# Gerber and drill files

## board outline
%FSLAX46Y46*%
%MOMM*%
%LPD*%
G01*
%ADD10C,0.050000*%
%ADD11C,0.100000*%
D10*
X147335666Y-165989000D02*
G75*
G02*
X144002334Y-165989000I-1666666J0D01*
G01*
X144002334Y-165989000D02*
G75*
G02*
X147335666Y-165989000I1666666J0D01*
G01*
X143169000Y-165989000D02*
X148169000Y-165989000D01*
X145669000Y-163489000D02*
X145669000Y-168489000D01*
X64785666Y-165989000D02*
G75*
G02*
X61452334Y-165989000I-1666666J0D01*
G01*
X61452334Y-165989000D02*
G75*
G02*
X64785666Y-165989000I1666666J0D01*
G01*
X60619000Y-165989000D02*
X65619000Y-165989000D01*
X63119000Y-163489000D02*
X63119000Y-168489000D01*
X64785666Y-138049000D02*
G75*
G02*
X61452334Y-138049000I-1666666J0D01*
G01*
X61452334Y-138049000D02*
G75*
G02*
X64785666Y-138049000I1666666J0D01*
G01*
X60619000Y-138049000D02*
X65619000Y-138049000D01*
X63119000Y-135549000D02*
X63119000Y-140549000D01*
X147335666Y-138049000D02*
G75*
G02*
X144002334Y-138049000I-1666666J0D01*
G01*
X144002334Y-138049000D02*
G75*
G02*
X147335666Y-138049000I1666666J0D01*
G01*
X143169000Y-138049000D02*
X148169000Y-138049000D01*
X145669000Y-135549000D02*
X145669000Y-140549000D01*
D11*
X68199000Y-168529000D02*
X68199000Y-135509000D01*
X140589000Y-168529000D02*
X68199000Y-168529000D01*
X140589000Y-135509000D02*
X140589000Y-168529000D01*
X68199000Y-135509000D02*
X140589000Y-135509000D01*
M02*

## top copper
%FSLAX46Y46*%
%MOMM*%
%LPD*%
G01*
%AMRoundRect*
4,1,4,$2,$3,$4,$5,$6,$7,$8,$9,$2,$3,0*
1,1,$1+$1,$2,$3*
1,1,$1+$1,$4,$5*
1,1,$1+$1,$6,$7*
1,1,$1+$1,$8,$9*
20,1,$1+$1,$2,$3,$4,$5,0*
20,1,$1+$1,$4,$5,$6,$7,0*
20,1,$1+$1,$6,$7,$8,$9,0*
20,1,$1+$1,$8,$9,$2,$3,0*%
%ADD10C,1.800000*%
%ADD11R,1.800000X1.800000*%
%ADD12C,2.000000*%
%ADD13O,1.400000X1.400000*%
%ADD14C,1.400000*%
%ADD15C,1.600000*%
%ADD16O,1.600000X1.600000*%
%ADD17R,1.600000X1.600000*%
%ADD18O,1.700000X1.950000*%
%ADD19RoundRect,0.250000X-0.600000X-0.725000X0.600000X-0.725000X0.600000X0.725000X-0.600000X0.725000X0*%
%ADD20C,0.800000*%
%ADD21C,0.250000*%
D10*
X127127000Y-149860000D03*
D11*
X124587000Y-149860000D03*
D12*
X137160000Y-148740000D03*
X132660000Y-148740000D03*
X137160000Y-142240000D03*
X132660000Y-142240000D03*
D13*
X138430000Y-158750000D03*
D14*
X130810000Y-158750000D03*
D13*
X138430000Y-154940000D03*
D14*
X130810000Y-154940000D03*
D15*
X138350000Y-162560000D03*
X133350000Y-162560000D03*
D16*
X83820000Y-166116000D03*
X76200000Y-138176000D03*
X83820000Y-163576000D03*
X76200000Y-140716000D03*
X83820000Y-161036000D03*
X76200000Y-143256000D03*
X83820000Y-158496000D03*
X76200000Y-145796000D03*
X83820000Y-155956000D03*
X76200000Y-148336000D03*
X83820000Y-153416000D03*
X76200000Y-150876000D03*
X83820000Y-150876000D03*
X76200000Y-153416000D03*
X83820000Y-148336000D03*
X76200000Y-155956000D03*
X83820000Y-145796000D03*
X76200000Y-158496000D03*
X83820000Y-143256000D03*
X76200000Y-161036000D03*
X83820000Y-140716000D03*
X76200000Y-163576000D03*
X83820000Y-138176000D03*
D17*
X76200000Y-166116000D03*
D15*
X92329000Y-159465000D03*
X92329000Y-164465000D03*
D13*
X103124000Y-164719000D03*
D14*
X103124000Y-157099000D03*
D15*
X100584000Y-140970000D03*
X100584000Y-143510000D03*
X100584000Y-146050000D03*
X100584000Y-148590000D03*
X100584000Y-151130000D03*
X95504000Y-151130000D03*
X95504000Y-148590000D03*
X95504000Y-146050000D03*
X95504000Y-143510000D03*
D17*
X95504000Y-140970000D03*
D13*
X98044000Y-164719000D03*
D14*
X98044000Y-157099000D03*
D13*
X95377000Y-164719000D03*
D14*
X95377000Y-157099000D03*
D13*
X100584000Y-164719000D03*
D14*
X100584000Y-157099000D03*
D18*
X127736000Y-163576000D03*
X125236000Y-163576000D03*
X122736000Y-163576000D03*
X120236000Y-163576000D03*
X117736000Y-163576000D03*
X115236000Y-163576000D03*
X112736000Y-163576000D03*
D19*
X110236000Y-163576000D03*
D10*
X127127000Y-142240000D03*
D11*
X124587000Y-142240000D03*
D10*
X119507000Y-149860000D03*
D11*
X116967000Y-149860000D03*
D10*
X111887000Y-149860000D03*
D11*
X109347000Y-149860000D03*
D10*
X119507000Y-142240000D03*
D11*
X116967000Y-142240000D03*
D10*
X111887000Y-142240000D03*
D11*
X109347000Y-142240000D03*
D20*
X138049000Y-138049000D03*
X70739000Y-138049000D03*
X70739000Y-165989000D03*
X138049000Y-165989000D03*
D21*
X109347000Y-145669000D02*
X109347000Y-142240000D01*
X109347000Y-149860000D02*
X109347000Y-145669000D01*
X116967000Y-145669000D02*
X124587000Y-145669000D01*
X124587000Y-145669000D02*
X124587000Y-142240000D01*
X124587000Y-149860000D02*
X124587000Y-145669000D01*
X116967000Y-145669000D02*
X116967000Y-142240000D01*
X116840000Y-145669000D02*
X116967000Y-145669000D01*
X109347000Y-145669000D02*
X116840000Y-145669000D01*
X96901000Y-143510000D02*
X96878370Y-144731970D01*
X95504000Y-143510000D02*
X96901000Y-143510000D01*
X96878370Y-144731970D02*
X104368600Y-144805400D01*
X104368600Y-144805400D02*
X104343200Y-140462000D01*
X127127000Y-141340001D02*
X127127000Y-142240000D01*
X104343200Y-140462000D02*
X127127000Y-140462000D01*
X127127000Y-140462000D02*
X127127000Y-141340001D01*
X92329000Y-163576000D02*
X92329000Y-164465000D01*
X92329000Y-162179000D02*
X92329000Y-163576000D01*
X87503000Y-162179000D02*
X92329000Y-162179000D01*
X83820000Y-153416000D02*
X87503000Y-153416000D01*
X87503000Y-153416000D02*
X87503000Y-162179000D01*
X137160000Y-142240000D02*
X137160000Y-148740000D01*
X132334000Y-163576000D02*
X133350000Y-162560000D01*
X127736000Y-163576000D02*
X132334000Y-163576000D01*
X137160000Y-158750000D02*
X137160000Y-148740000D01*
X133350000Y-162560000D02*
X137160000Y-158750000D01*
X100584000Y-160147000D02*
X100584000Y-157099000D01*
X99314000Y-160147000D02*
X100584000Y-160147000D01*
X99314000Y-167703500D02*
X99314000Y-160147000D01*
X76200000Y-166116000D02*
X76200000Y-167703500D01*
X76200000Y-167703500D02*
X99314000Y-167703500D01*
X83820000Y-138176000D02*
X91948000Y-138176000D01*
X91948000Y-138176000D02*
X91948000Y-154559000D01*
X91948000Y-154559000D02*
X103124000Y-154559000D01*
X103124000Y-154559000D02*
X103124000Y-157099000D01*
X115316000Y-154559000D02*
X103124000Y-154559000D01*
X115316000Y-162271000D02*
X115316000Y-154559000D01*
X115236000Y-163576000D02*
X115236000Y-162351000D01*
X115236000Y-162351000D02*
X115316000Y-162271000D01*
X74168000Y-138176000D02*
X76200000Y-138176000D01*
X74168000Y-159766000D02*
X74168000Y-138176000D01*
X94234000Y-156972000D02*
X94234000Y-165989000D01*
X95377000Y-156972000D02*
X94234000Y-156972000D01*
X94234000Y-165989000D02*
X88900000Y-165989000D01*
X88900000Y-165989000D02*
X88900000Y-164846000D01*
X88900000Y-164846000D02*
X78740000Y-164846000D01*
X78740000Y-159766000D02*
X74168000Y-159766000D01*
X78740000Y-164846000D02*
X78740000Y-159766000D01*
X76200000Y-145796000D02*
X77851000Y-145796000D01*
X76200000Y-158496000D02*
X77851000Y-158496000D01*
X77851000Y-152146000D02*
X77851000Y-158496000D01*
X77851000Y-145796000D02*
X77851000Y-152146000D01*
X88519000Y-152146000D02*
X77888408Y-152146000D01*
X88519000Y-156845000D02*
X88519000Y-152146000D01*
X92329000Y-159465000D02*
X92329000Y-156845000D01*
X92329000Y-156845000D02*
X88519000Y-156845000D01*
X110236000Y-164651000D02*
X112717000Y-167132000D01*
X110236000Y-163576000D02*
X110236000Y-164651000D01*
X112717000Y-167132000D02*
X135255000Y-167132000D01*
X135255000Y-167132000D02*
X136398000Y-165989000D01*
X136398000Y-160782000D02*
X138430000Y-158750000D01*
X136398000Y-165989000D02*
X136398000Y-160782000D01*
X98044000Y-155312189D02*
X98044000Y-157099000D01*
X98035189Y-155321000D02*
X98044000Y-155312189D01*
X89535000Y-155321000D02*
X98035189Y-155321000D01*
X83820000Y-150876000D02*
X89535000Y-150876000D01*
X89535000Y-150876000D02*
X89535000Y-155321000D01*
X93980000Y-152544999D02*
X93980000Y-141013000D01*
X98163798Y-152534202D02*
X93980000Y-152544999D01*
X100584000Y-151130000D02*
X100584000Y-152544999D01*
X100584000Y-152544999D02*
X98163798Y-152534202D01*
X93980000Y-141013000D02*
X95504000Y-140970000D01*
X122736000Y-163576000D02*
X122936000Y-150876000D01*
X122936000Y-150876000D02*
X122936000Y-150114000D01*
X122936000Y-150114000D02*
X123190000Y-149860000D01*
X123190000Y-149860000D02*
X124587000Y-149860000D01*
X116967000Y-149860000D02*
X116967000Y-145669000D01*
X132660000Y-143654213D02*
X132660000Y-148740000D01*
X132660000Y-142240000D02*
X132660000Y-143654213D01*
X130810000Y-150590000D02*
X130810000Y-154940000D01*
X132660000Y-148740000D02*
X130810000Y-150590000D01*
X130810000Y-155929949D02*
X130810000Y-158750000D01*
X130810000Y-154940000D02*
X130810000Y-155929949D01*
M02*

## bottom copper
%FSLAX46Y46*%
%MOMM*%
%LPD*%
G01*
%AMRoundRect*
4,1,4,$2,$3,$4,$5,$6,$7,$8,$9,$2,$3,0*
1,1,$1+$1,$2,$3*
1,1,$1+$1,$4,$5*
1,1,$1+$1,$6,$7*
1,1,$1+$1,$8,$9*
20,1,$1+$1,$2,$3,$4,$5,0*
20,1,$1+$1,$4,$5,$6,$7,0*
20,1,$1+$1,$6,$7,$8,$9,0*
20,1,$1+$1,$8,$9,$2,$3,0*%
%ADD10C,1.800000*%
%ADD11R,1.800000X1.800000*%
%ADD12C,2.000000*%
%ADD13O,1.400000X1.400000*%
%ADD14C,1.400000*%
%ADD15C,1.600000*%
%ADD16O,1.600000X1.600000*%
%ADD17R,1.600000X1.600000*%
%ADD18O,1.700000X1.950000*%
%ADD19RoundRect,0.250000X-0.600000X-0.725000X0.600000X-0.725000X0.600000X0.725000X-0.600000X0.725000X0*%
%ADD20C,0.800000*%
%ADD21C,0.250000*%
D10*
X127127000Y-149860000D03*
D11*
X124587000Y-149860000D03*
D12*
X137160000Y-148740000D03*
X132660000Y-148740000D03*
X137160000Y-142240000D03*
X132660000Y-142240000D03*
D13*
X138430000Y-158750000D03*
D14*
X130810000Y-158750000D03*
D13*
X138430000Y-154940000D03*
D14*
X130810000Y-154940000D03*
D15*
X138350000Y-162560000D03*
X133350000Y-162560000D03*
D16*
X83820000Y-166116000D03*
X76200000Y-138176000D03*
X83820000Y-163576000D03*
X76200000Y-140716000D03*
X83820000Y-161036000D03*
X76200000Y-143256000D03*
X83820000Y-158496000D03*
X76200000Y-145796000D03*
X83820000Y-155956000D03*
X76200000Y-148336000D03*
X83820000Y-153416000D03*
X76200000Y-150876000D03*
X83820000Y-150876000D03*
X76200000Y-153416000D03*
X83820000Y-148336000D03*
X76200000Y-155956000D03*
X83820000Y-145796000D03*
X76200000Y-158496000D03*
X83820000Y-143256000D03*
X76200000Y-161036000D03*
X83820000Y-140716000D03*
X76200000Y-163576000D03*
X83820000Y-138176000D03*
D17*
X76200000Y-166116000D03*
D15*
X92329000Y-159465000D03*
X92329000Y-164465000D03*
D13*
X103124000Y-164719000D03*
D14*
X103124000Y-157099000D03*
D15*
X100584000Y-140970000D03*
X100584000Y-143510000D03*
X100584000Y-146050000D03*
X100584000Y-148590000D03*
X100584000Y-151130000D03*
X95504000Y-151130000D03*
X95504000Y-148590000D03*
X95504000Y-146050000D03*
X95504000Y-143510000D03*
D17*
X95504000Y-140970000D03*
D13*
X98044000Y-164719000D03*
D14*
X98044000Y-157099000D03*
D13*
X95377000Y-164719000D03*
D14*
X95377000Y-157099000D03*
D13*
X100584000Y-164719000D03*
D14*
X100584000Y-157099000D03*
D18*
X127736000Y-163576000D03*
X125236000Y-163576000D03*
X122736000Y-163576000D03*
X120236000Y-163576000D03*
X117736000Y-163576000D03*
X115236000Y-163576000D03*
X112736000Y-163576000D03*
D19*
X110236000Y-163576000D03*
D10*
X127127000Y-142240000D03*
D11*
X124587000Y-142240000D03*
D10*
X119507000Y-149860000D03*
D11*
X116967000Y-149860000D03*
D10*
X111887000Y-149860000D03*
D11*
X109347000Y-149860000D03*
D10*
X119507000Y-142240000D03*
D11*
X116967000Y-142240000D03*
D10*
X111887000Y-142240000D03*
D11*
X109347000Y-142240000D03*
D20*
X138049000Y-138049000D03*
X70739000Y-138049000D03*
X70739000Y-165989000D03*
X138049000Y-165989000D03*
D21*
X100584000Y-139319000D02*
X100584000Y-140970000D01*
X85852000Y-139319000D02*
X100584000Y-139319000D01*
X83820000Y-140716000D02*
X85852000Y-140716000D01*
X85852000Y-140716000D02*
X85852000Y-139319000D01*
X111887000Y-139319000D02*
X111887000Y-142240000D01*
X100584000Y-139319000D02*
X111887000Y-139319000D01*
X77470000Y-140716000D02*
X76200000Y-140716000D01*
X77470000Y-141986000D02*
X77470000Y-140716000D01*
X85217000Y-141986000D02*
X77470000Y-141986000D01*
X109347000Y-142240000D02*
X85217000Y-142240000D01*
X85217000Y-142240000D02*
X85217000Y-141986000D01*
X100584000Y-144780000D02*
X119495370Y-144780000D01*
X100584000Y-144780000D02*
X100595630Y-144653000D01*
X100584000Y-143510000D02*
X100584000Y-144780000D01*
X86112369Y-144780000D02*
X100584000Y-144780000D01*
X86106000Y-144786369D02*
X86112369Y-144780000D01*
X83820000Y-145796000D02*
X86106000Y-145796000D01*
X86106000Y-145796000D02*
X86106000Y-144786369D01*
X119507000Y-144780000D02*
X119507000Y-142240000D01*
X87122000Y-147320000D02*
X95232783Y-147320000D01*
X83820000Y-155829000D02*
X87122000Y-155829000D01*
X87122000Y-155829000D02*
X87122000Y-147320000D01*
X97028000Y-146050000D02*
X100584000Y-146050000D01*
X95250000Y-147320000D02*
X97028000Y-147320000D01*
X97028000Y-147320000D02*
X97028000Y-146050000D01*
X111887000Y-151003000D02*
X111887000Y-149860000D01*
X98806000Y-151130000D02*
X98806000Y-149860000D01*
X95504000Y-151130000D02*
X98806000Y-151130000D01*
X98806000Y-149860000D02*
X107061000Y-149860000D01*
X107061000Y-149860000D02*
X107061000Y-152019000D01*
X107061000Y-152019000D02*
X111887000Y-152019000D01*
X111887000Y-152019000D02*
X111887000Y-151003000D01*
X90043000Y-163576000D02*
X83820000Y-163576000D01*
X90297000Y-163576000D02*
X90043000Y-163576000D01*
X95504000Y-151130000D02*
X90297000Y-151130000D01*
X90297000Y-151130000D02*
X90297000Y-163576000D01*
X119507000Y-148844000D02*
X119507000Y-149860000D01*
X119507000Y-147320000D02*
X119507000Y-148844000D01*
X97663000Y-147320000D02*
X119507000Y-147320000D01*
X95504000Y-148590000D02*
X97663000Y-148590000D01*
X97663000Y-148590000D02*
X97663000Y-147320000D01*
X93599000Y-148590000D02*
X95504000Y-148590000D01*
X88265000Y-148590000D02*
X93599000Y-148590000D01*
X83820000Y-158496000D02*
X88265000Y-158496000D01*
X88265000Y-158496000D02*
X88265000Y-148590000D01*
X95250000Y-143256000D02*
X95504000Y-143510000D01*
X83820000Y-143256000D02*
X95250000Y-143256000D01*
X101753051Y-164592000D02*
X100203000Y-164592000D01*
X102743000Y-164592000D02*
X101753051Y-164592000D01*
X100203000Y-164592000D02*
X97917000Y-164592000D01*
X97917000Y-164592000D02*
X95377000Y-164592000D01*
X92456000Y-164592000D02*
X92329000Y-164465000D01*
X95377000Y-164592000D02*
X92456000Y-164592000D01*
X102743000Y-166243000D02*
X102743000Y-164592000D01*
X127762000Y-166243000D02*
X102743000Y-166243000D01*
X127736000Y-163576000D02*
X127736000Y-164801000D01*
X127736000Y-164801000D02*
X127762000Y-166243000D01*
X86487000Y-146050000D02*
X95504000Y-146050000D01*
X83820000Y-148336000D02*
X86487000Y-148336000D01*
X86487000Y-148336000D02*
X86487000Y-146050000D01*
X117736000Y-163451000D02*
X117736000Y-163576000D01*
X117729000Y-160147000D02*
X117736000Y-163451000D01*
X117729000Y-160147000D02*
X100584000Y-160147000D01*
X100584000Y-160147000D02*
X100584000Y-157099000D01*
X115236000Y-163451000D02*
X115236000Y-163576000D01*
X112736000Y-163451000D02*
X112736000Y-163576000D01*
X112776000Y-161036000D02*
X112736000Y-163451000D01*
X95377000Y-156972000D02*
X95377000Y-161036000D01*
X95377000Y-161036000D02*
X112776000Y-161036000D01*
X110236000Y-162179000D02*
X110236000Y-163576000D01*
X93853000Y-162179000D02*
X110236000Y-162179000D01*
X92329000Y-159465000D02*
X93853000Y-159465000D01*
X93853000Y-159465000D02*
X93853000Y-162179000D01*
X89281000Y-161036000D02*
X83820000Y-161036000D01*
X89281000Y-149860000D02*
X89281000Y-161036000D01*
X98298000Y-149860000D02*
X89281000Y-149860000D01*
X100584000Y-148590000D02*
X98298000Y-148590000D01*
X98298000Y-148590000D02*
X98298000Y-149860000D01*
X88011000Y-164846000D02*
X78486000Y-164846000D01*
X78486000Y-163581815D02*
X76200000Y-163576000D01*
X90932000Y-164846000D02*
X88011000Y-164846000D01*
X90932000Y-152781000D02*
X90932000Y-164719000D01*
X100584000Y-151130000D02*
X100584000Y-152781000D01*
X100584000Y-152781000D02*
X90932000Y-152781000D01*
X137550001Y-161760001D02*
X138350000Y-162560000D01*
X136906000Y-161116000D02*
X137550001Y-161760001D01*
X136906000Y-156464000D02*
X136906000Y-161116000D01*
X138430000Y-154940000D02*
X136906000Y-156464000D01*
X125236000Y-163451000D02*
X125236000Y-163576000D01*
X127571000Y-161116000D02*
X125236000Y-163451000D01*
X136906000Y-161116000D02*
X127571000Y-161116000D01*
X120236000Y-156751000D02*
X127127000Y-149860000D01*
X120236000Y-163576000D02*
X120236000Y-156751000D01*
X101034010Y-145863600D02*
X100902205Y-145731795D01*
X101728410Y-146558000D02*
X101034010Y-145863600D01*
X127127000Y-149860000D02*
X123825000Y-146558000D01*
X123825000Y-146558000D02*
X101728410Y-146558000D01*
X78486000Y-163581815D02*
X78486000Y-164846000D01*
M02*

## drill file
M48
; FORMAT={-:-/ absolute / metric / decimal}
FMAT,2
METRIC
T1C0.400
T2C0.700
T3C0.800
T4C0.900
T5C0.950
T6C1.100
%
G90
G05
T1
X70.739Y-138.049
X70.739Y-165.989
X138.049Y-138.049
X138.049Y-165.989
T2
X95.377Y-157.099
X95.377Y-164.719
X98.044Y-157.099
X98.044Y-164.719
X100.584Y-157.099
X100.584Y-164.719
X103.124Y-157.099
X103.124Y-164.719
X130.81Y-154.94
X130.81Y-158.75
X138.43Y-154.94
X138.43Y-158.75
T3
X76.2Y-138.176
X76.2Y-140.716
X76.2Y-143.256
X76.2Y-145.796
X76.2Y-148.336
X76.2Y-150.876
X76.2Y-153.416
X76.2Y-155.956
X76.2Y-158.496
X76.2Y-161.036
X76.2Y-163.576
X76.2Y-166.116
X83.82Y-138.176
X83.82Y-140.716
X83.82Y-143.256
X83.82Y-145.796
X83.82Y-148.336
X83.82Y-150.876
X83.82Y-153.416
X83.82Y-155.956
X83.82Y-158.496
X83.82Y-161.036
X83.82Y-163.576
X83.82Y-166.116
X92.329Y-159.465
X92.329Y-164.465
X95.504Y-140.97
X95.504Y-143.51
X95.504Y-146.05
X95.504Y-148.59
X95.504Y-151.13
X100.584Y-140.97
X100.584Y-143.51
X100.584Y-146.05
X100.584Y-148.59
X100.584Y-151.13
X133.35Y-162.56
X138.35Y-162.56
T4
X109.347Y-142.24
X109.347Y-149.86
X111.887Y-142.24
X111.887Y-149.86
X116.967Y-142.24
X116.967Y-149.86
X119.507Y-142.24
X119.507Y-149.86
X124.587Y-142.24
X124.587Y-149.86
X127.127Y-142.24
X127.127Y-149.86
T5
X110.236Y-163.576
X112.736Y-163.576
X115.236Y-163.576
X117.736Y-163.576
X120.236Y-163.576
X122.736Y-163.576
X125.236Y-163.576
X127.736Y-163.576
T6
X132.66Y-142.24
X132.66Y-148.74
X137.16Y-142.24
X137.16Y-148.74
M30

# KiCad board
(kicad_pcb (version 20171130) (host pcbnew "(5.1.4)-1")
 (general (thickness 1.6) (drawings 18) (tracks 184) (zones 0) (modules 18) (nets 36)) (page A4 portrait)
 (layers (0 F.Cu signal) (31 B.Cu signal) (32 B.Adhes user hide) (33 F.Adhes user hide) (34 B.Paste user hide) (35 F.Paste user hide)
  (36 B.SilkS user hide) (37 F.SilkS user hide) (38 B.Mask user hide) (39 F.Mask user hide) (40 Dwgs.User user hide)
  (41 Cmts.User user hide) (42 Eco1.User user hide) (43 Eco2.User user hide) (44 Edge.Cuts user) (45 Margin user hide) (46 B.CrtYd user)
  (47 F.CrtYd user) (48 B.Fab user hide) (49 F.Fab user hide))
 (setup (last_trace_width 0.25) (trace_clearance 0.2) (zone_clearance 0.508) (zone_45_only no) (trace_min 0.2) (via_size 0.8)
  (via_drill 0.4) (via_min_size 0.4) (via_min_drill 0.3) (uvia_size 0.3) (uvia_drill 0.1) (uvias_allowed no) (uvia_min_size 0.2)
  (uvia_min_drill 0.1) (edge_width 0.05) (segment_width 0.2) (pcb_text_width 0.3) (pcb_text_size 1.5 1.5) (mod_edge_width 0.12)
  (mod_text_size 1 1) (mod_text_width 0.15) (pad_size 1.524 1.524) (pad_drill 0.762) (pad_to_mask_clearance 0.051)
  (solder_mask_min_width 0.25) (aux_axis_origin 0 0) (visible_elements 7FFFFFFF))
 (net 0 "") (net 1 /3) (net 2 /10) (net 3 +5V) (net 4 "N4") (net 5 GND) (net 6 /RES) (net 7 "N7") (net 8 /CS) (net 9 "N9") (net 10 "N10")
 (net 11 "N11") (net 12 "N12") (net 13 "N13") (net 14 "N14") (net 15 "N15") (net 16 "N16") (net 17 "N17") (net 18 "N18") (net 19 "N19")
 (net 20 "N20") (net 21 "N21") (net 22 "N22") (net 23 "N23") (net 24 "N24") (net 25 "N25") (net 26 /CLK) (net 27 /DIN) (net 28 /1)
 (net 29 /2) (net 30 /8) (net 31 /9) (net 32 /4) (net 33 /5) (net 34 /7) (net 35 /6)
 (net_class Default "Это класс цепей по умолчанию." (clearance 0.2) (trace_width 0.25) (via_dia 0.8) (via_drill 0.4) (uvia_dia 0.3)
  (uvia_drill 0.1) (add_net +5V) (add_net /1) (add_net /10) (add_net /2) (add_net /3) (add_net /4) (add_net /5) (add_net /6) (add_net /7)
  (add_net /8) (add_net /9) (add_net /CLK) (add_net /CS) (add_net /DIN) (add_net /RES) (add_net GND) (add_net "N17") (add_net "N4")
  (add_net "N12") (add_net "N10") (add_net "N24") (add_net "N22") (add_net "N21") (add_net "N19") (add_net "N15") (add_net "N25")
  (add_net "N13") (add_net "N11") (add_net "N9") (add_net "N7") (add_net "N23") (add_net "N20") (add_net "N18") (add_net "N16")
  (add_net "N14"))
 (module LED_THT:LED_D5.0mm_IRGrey (layer F.Cu) (at 124.587 149.86)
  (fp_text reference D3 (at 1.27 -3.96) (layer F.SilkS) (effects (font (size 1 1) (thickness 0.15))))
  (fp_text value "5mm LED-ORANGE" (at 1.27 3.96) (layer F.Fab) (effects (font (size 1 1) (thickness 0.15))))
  (pad 2 thru_hole circle (at 2.54 0) (size 1.8 1.8) (drill 0.9) (layers *.Cu *.Mask) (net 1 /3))
  (pad 1 thru_hole rect (at 0 0) (size 1.8 1.8) (drill 0.9) (layers *.Cu *.Mask) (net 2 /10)))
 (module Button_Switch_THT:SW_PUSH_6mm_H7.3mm (layer F.Cu) (at 137.16 142.24 270)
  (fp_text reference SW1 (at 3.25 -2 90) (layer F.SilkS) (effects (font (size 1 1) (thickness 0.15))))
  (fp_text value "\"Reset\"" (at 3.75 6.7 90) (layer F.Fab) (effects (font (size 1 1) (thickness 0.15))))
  (pad 1 thru_hole circle (at 6.5 0) (size 2 2) (drill 1.1) (layers *.Cu *.Mask) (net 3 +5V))
  (pad 2 thru_hole circle (at 6.5 4.5) (size 2 2) (drill 1.1) (layers *.Cu *.Mask) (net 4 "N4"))
  (pad 1 thru_hole circle (at 0 0) (size 2 2) (drill 1.1) (layers *.Cu *.Mask) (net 3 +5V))
  (pad 2 thru_hole circle (at 0 4.5) (size 2 2) (drill 1.1) (layers *.Cu *.Mask) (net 4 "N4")))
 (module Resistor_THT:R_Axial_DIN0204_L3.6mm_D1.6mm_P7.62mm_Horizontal (layer B.Cu) (at 130.81 158.75)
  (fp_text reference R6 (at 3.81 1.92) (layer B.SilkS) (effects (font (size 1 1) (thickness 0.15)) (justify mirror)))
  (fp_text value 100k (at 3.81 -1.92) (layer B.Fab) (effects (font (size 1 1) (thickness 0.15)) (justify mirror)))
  (pad 2 thru_hole oval (at 7.62 0) (size 1.4 1.4) (drill 0.7) (layers *.Cu *.Mask) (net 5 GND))
  (pad 1 thru_hole circle (at 0 0) (size 1.4 1.4) (drill 0.7) (layers *.Cu *.Mask) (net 4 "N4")))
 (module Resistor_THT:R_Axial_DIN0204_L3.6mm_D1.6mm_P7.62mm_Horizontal (layer B.Cu) (at 130.81 154.94)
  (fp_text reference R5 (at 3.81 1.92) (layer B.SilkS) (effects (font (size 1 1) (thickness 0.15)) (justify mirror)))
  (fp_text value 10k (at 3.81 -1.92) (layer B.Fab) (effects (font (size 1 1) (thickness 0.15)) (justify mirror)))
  (pad 2 thru_hole oval (at 7.62 0) (size 1.4 1.4) (drill 0.7) (layers *.Cu *.Mask) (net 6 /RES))
  (pad 1 thru_hole circle (at 0 0) (size 1.4 1.4) (drill 0.7) (layers *.Cu *.Mask) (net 4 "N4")))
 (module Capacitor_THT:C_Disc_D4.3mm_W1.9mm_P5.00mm (layer B.Cu) (at 133.35 162.56)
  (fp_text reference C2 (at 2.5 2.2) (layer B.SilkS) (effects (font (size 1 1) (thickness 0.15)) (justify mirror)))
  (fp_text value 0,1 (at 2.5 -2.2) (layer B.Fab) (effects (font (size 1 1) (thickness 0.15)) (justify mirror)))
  (pad 2 thru_hole circle (at 5 0) (size 1.6 1.6) (drill 0.8) (layers *.Cu *.Mask) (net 6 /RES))
  (pad 1 thru_hole circle (at 0 0) (size 1.6 1.6) (drill 0.8) (layers *.Cu *.Mask) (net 3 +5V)))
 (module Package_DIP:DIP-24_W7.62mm (layer B.Cu) (at 76.2 166.116)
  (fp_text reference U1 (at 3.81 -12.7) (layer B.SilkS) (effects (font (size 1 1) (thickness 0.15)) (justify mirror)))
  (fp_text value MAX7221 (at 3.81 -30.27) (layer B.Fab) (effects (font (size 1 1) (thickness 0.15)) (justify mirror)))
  (pad 24 thru_hole oval (at 7.62 0) (size 1.6 1.6) (drill 0.8) (layers *.Cu *.Mask) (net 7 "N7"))
  (pad 12 thru_hole oval (at 0 -27.94) (size 1.6 1.6) (drill 0.8) (layers *.Cu *.Mask) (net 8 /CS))
  (pad 23 thru_hole oval (at 7.62 -2.54) (size 1.6 1.6) (drill 0.8) (layers *.Cu *.Mask) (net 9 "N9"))
  (pad 11 thru_hole oval (at 0 -25.4) (size 1.6 1.6) (drill 0.8) (layers *.Cu *.Mask) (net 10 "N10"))
  (pad 22 thru_hole oval (at 7.62 -5.08) (size 1.6 1.6) (drill 0.8) (layers *.Cu *.Mask) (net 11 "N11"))
  (pad 10 thru_hole oval (at 0 -22.86) (size 1.6 1.6) (drill 0.8) (layers *.Cu *.Mask) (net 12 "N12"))
  (pad 21 thru_hole oval (at 7.62 -7.62) (size 1.6 1.6) (drill 0.8) (layers *.Cu *.Mask) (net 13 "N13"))
  (pad 9 thru_hole oval (at 0 -20.32) (size 1.6 1.6) (drill 0.8) (layers *.Cu *.Mask) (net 5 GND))
  (pad 20 thru_hole oval (at 7.62 -10.16) (size 1.6 1.6) (drill 0.8) (layers *.Cu *.Mask) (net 1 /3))
  (pad 8 thru_hole oval (at 0 -17.78) (size 1.6 1.6) (drill 0.8) (layers *.Cu *.Mask) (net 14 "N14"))
  (pad 19 thru_hole oval (at 7.62 -12.7) (size 1.6 1.6) (drill 0.8) (layers *.Cu *.Mask) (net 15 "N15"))
  (pad 7 thru_hole oval (at 0 -15.24) (size 1.6 1.6) (drill 0.8) (layers *.Cu *.Mask) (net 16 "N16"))
  (pad 18 thru_hole oval (at 7.62 -15.24) (size 1.6 1.6) (drill 0.8) (layers *.Cu *.Mask) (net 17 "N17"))
  (pad 6 thru_hole oval (at 0 -12.7) (size 1.6 1.6) (drill 0.8) (layers *.Cu *.Mask) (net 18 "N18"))
  (pad 17 thru_hole oval (at 7.62 -17.78) (size 1.6 1.6) (drill 0.8) (layers *.Cu *.Mask) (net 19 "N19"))
  (pad 5 thru_hole oval (at 0 -10.16) (size 1.6 1.6) (drill 0.8) (layers *.Cu *.Mask) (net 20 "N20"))
  (pad 16 thru_hole oval (at 7.62 -20.32) (size 1.6 1.6) (drill 0.8) (layers *.Cu *.Mask) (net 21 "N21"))
  (pad 4 thru_hole oval (at 0 -7.62) (size 1.6 1.6) (drill 0.8) (layers *.Cu *.Mask) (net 5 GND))
  (pad 15 thru_hole oval (at 7.62 -22.86) (size 1.6 1.6) (drill 0.8) (layers *.Cu *.Mask) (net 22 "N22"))
  (pad 3 thru_hole oval (at 0 -5.08) (size 1.6 1.6) (drill 0.8) (layers *.Cu *.Mask) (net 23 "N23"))
  (pad 14 thru_hole oval (at 7.62 -25.4) (size 1.6 1.6) (drill 0.8) (layers *.Cu *.Mask) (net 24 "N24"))
  (pad 2 thru_hole oval (at 0 -2.54) (size 1.6 1.6) (drill 0.8) (layers *.Cu *.Mask) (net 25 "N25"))
  (pad 13 thru_hole oval (at 7.62 -27.94) (size 1.6 1.6) (drill 0.8) (layers *.Cu *.Mask) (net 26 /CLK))
  (pad 1 thru_hole rect (at 0 0) (size 1.6 1.6) (drill 0.8) (layers *.Cu *.Mask) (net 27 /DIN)))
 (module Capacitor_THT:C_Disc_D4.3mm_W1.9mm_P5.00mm (layer B.Cu) (at 92.329 164.465 90)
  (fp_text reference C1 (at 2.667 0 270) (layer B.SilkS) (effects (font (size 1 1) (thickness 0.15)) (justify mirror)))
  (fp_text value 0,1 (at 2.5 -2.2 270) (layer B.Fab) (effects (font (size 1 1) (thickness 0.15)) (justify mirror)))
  (pad 2 thru_hole circle (at 5 0 90) (size 1.6 1.6) (drill 0.8) (layers *.Cu *.Mask) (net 5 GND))
  (pad 1 thru_hole circle (at 0 0 90) (size 1.6 1.6) (drill 0.8) (layers *.Cu *.Mask) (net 3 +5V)))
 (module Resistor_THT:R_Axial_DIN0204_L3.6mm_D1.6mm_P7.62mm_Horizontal (layer B.Cu) (at 103.124 157.099 270)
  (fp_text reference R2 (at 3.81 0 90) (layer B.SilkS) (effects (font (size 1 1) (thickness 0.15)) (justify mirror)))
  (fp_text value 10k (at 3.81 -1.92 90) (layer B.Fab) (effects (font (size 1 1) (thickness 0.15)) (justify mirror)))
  (pad 2 thru_hole oval (at 7.62 0 270) (size 1.4 1.4) (drill 0.7) (layers *.Cu *.Mask) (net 3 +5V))
  (pad 1 thru_hole circle (at 0 0 270) (size 1.4 1.4) (drill 0.7) (layers *.Cu *.Mask) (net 26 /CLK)))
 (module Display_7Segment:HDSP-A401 (layer F.Cu) (at 95.504 140.97)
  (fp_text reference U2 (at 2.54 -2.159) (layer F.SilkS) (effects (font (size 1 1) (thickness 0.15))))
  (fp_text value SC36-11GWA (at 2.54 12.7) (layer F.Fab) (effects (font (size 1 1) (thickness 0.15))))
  (pad 10 thru_hole circle (at 5.08 0) (size 1.6 1.6) (drill 0.8) (layers *.Cu *.Mask) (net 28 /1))
  (pad 9 thru_hole circle (at 5.08 2.54) (size 1.6 1.6) (drill 0.8) (layers *.Cu *.Mask) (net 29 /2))
  (pad 8 thru_hole circle (at 5.08 5.08) (size 1.6 1.6) (drill 0.8) (layers *.Cu *.Mask) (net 1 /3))
  (pad 7 thru_hole circle (at 5.08 7.62) (size 1.6 1.6) (drill 0.8) (layers *.Cu *.Mask) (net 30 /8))
  (pad 6 thru_hole circle (at 5.08 10.16) (size 1.6 1.6) (drill 0.8) (layers *.Cu *.Mask) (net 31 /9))
  (pad 5 thru_hole circle (at 0 10.16) (size 1.6 1.6) (drill 0.8) (layers *.Cu *.Mask) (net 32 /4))
  (pad 4 thru_hole circle (at 0 7.62) (size 1.6 1.6) (drill 0.8) (layers *.Cu *.Mask) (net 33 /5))
  (pad 3 thru_hole circle (at 0 5.08) (size 1.6 1.6) (drill 0.8) (layers *.Cu *.Mask) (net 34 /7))
  (pad 2 thru_hole circle (at 0 2.54) (size 1.6 1.6) (drill 0.8) (layers *.Cu *.Mask) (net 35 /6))
  (pad 1 thru_hole rect (at 0 0) (size 1.6 1.6) (drill 0.8) (layers *.Cu *.Mask) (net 31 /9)))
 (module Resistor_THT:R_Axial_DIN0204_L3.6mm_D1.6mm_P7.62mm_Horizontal (layer B.Cu) (at 98.044 157.099 270)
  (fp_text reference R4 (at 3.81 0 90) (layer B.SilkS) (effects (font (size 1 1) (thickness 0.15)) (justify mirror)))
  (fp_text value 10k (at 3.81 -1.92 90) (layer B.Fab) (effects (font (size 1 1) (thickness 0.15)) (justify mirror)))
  (pad 2 thru_hole oval (at 7.62 0 270) (size 1.4 1.4) (drill 0.7) (layers *.Cu *.Mask) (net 3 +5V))
  (pad 1 thru_hole circle (at 0 0 270) (size 1.4 1.4) (drill 0.7) (layers *.Cu *.Mask) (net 17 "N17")))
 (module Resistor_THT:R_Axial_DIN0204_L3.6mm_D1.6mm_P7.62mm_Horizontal (layer B.Cu) (at 95.377 157.099 270)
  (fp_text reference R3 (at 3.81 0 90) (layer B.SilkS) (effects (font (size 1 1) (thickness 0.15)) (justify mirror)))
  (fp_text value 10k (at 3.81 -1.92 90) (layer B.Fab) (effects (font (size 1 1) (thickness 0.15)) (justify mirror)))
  (pad 2 thru_hole oval (at 7.62 0 270) (size 1.4 1.4) (drill 0.7) (layers *.Cu *.Mask) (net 3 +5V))
  (pad 1 thru_hole circle (at 0 0 270) (size 1.4 1.4) (drill 0.7) (layers *.Cu *.Mask) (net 8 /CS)))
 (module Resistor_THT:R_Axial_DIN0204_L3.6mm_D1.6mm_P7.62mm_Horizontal (layer B.Cu) (at 100.584 157.099 270)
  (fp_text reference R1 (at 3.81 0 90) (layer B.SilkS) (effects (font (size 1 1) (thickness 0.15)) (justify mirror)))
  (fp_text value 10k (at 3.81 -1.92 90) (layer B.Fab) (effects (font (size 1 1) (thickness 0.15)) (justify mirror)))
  (pad 2 thru_hole oval (at 7.62 0 270) (size 1.4 1.4) (drill 0.7) (layers *.Cu *.Mask) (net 3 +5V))
  (pad 1 thru_hole circle (at 0 0 270) (size 1.4 1.4) (drill 0.7) (layers *.Cu *.Mask) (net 27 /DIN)))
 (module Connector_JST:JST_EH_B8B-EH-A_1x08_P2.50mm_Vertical (layer F.Cu) (at 110.236 163.576)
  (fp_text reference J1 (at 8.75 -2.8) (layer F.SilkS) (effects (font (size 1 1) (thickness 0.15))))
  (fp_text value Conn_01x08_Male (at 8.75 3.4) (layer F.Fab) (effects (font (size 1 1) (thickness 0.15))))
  (pad 8 thru_hole oval (at 17.5 0) (size 1.7 1.95) (drill 0.95) (layers *.Cu *.Mask) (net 3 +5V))
  (pad 7 thru_hole oval (at 15 0) (size 1.7 1.95) (drill 0.95) (layers *.Cu *.Mask) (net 6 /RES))
  (pad 6 thru_hole oval (at 12.5 0) (size 1.7 1.95) (drill 0.95) (layers *.Cu *.Mask) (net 2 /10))
  (pad 5 thru_hole oval (at 10 0) (size 1.7 1.95) (drill 0.95) (layers *.Cu *.Mask) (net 1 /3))
  (pad 4 thru_hole oval (at 7.5 0) (size 1.7 1.95) (drill 0.95) (layers *.Cu *.Mask) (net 27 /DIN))
  (pad 3 thru_hole oval (at 5 0) (size 1.7 1.95) (drill 0.95) (layers *.Cu *.Mask) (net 26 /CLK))
  (pad 2 thru_hole oval (at 2.5 0) (size 1.7 1.95) (drill 0.95) (layers *.Cu *.Mask) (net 8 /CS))
  (pad 1 thru_hole roundrect (at 0 0) (size 1.7 1.95) (drill 0.95) (layers *.Cu *.Mask) (roundrect_rratio 0.147059) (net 5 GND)))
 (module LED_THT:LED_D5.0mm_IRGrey (layer F.Cu) (at 124.587 142.24)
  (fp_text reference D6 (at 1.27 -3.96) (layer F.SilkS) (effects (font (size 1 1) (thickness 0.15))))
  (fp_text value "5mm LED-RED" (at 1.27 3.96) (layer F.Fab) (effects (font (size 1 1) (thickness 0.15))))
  (pad 2 thru_hole circle (at 2.54 0) (size 1.8 1.8) (drill 0.9) (layers *.Cu *.Mask) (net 35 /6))
  (pad 1 thru_hole rect (at 0 0) (size 1.8 1.8) (drill 0.9) (layers *.Cu *.Mask) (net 2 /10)))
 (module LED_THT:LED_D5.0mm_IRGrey (layer F.Cu) (at 116.967 149.86)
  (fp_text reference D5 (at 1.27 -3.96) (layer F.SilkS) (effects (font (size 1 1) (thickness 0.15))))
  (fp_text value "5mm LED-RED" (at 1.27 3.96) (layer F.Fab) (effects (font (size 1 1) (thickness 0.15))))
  (pad 2 thru_hole circle (at 2.54 0) (size 1.8 1.8) (drill 0.9) (layers *.Cu *.Mask) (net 33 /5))
  (pad 1 thru_hole rect (at 0 0) (size 1.8 1.8) (drill 0.9) (layers *.Cu *.Mask) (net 2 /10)))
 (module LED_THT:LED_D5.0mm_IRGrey (layer F.Cu) (at 109.347 149.86)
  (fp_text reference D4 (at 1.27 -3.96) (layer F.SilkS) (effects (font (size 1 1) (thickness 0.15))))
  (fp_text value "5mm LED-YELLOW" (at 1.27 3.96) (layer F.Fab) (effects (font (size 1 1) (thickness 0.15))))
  (pad 2 thru_hole circle (at 2.54 0) (size 1.8 1.8) (drill 0.9) (layers *.Cu *.Mask) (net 32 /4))
  (pad 1 thru_hole rect (at 0 0) (size 1.8 1.8) (drill 0.9) (layers *.Cu *.Mask) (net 2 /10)))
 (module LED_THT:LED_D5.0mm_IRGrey (layer F.Cu) (at 116.967 142.24)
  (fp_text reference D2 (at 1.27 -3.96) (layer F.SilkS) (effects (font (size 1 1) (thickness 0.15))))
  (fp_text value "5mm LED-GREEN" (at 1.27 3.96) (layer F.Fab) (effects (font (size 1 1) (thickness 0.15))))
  (pad 2 thru_hole circle (at 2.54 0) (size 1.8 1.8) (drill 0.9) (layers *.Cu *.Mask) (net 29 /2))
  (pad 1 thru_hole rect (at 0 0) (size 1.8 1.8) (drill 0.9) (layers *.Cu *.Mask) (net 2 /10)))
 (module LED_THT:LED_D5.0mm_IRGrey (layer F.Cu) (at 109.347 142.24)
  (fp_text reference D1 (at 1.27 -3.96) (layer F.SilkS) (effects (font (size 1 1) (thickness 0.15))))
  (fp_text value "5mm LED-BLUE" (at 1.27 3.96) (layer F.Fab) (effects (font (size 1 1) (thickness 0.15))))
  (pad 2 thru_hole circle (at 2.54 0) (size 1.8 1.8) (drill 0.9) (layers *.Cu *.Mask) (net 28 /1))
  (pad 1 thru_hole rect (at 0 0) (size 1.8 1.8) (drill 0.9) (layers *.Cu *.Mask) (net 2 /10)))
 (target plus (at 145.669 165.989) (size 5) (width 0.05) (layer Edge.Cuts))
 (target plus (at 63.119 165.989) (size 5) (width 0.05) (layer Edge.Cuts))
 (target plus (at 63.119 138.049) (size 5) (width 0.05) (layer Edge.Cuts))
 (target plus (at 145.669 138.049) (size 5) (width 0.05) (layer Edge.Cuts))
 (gr_line (start 68.199 168.529) (end 68.199 135.509) (layer Edge.Cuts) (width 0.1))
 (gr_line (start 140.589 168.529) (end 68.199 168.529) (layer Edge.Cuts) (width 0.1))
 (gr_line (start 140.589 135.509) (end 140.589 168.529) (layer Edge.Cuts) (width 0.1))
 (gr_line (start 68.199 135.509) (end 140.589 135.509) (layer Edge.Cuts) (width 0.1))
 (via (at 138.049 138.049) (size 0.8) (drill 0.4) (layers F.Cu B.Cu) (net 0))
 (via (at 70.739 138.049) (size 0.8) (drill 0.4) (layers F.Cu B.Cu) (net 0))
 (via (at 70.739 165.989) (size 0.8) (drill 0.4) (layers F.Cu B.Cu) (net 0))
 (via (at 138.049 165.989) (size 0.8) (drill 0.4) (layers F.Cu B.Cu) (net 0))
 (segment (start 100.584 139.319) (end 100.584 140.97) (width 0.25) (layer B.Cu) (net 28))
 (segment (start 85.852 139.319) (end 100.584 139.319) (width 0.25) (layer B.Cu) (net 28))
 (segment (start 83.82 140.716) (end 85.852 140.716) (width 0.25) (layer B.Cu) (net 28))
 (segment (start 85.852 140.716) (end 85.852 139.319) (width 0.25) (layer B.Cu) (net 28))
 (segment (start 111.887 139.319) (end 111.887 142.24) (width 0.25) (layer B.Cu) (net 28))
 (segment (start 100.584 139.319) (end 111.887 139.319) (width 0.25) (layer B.Cu) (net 28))
 (segment (start 109.347 145.669) (end 109.347 142.24) (width 0.25) (layer F.Cu) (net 2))
 (segment (start 109.347 149.86) (end 109.347 145.669) (width 0.25) (layer F.Cu) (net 2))
 (segment (start 116.967 145.669) (end 124.587 145.669) (width 0.25) (layer F.Cu) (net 2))
 (segment (start 124.587 145.669) (end 124.587 142.24) (width 0.25) (layer F.Cu) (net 2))
 (segment (start 124.587 149.86) (end 124.587 145.669) (width 0.25) (layer F.Cu) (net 2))
 (segment (start 116.967 145.669) (end 116.967 142.24) (width 0.25) (layer F.Cu) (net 2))
 (segment (start 77.47 140.716) (end 76.2 140.716) (width 0.25) (layer B.Cu) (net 2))
 (segment (start 77.47 141.986) (end 77.47 140.716) (width 0.25) (layer B.Cu) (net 2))
 (segment (start 85.217 141.986) (end 77.47 141.986) (width 0.25) (layer B.Cu) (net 2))
 (segment (start 109.347 142.24) (end 85.217 142.24) (width 0.25) (layer B.Cu) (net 2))
 (segment (start 85.217 142.24) (end 85.217 141.986) (width 0.25) (layer B.Cu) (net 2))
 (segment (start 116.84 145.669) (end 116.967 145.669) (width 0.25) (layer F.Cu) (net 2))
 (segment (start 109.347 145.669) (end 116.84 145.669) (width 0.25) (layer F.Cu) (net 2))
 (segment (start 100.584 144.78) (end 119.49537 144.78) (width 0.25) (layer B.Cu) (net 29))
 (segment (start 100.584 144.78) (end 100.59563 144.653) (width 0.25) (layer B.Cu) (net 29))
 (segment (start 100.584 143.51) (end 100.584 144.78) (width 0.25) (layer B.Cu) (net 29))
 (segment (start 86.112369 144.78) (end 100.584 144.78) (width 0.25) (layer B.Cu) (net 29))
 (segment (start 86.106 144.786369) (end 86.112369 144.78) (width 0.25) (layer B.Cu) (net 29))
 (segment (start 83.82 145.796) (end 86.106 145.796) (width 0.25) (layer B.Cu) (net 29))
 (segment (start 86.106 145.796) (end 86.106 144.786369) (width 0.25) (layer B.Cu) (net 29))
 (segment (start 119.507 144.78) (end 119.507 142.24) (width 0.25) (layer B.Cu) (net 29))
 (segment (start 87.122 147.32) (end 95.232783 147.32) (width 0.25) (layer B.Cu) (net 1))
 (segment (start 83.82 155.829) (end 87.122 155.829) (width 0.25) (layer B.Cu) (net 1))
 (segment (start 87.122 155.829) (end 87.122 147.32) (width 0.25) (layer B.Cu) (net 1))
 (segment (start 97.028 146.05) (end 100.584 146.05) (width 0.25) (layer B.Cu) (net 1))
 (segment (start 95.25 147.32) (end 97.028 147.32) (width 0.25) (layer B.Cu) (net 1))
 (segment (start 97.028 147.32) (end 97.028 146.05) (width 0.25) (layer B.Cu) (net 1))
 (segment (start 111.887 151.003) (end 111.887 149.86) (width 0.25) (layer B.Cu) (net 32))
 (segment (start 98.806 151.13) (end 98.806 149.86) (width 0.25) (layer B.Cu) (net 32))
 (segment (start 95.504 151.13) (end 98.806 151.13) (width 0.25) (layer B.Cu) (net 32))
 (segment (start 98.806 149.86) (end 107.061 149.86) (width 0.25) (layer B.Cu) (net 32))
 (segment (start 107.061 149.86) (end 107.061 152.019) (width 0.25) (layer B.Cu) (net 32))
 (segment (start 107.061 152.019) (end 111.887 152.019) (width 0.25) (layer B.Cu) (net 32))
 (segment (start 111.887 152.019) (end 111.887 151.003) (width 0.25) (layer B.Cu) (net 32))
 (segment (start 90.043 163.576) (end 83.82 163.576) (width 0.25) (layer B.Cu) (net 32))
 (segment (start 90.297 163.576) (end 90.043 163.576) (width 0.25) (layer B.Cu) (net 32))
 (segment (start 95.504 151.13) (end 90.297 151.13) (width 0.25) (layer B.Cu) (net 32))
 (segment (start 90.297 151.13) (end 90.297 163.576) (width 0.25) (layer B.Cu) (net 32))
 (segment (start 119.507 148.844) (end 119.507 149.86) (width 0.25) (layer B.Cu) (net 33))
 (segment (start 119.507 147.32) (end 119.507 148.844) (width 0.25) (layer B.Cu) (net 33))
 (segment (start 97.663 147.32) (end 119.507 147.32) (width 0.25) (layer B.Cu) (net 33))
 (segment (start 95.504 148.59) (end 97.663 148.59) (width 0.25) (layer B.Cu) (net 33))
 (segment (start 97.663 148.59) (end 97.663 147.32) (width 0.25) (layer B.Cu) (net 33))
 (segment (start 93.599 148.59) (end 95.504 148.59) (width 0.25) (layer B.Cu) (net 33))
 (segment (start 88.265 148.59) (end 93.599 148.59) (width 0.25) (layer B.Cu) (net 33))
 (segment (start 83.82 158.496) (end 88.265 158.496) (width 0.25) (layer B.Cu) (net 33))
 (segment (start 88.265 158.496) (end 88.265 148.59) (width 0.25) (layer B.Cu) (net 33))
 (segment (start 95.25 143.256) (end 95.504 143.51) (width 0.25) (layer B.Cu) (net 35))
 (segment (start 83.82 143.256) (end 95.25 143.256) (width 0.25) (layer B.Cu) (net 35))
 (segment (start 96.901 143.51) (end 96.87837 144.73197) (width 0.25) (layer F.Cu) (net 35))
 (segment (start 95.504 143.51) (end 96.901 143.51) (width 0.25) (layer F.Cu) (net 35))
 (segment (start 96.87837 144.73197) (end 104.3686 144.8054) (width 0.25) (layer F.Cu) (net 35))
 (segment (start 104.3686 144.8054) (end 104.3432 140.462) (width 0.25) (layer F.Cu) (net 35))
 (segment (start 127.127 141.340001) (end 127.127 142.24) (width 0.25) (layer F.Cu) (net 35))
 (segment (start 104.3432 140.462) (end 127.127 140.462) (width 0.25) (layer F.Cu) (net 35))
 (segment (start 127.127 140.462) (end 127.127 141.340001) (width 0.25) (layer F.Cu) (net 35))
 (segment (start 101.753051 164.592) (end 100.203 164.592) (width 0.25) (layer B.Cu) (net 3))
 (segment (start 102.743 164.592) (end 101.753051 164.592) (width 0.25) (layer B.Cu) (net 3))
 (segment (start 100.203 164.592) (end 97.917 164.592) (width 0.25) (layer B.Cu) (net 3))
 (segment (start 97.917 164.592) (end 95.377 164.592) (width 0.25) (layer B.Cu) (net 3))
 (segment (start 92.456 164.592) (end 92.329 164.465) (width 0.25) (layer B.Cu) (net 3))
 (segment (start 95.377 164.592) (end 92.456 164.592) (width 0.25) (layer B.Cu) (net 3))
 (segment (start 102.743 166.243) (end 102.743 164.592) (width 0.25) (layer B.Cu) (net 3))
 (segment (start 127.762 166.243) (end 102.743 166.243) (width 0.25) (layer B.Cu) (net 3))
 (segment (start 127.736 163.576) (end 127.736 164.801) (width 0.25) (layer B.Cu) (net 3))
 (segment (start 127.736 164.801) (end 127.762 166.243) (width 0.25) (layer B.Cu) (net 3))
 (segment (start 92.329 163.576) (end 92.329 164.465) (width 0.25) (layer F.Cu) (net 3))
 (segment (start 92.329 162.179) (end 92.329 163.576) (width 0.25) (layer F.Cu) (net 3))
 (segment (start 87.503 162.179) (end 92.329 162.179) (width 0.25) (layer F.Cu) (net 3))
 (segment (start 83.82 153.416) (end 87.503 153.416) (width 0.25) (layer F.Cu) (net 3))
 (segment (start 87.503 153.416) (end 87.503 162.179) (width 0.25) (layer F.Cu) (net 3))
 (segment (start 137.16 142.24) (end 137.16 148.74) (width 0.25) (layer F.Cu) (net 3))
 (segment (start 132.334 163.576) (end 133.35 162.56) (width 0.25) (layer F.Cu) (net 3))
 (segment (start 127.736 163.576) (end 132.334 163.576) (width 0.25) (layer F.Cu) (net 3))
 (segment (start 137.16 158.75) (end 137.16 148.74) (width 0.25) (layer F.Cu) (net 3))
 (segment (start 133.35 162.56) (end 137.16 158.75) (width 0.25) (layer F.Cu) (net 3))
 (segment (start 86.487 146.05) (end 95.504 146.05) (width 0.25) (layer B.Cu) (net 34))
 (segment (start 83.82 148.336) (end 86.487 148.336) (width 0.25) (layer B.Cu) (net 34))
 (segment (start 86.487 148.336) (end 86.487 146.05) (width 0.25) (layer B.Cu) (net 34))
 (segment (start 117.736 163.451) (end 117.736 163.576) (width 0.25) (layer B.Cu) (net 27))
 (segment (start 117.729 160.147) (end 117.736 163.451) (width 0.25) (layer B.Cu) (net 27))
 (segment (start 117.729 160.147) (end 100.584 160.147) (width 0.25) (layer B.Cu) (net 27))
 (segment (start 100.584 160.147) (end 100.584 157.099) (width 0.25) (layer B.Cu) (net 27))
 (segment (start 100.584 160.147) (end 100.584 157.099) (width 0.25) (layer F.Cu) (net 27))
 (segment (start 99.314 160.147) (end 100.584 160.147) (width 0.25) (layer F.Cu) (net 27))
 (segment (start 99.314 167.7035) (end 99.314 160.147) (width 0.25) (layer F.Cu) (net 27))
 (segment (start 76.2 166.116) (end 76.2 167.7035) (width 0.25) (layer F.Cu) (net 27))
 (segment (start 76.2 167.7035) (end 99.314 167.7035) (width 0.25) (layer F.Cu) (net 27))
 (segment (start 115.236 163.451) (end 115.236 163.576) (width 0.25) (layer B.Cu) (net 26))
 (segment (start 83.82 138.176) (end 91.948 138.176) (width 0.25) (layer F.Cu) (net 26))
 (segment (start 91.948 138.176) (end 91.948 154.559) (width 0.25) (layer F.Cu) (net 26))
 (segment (start 91.948 154.559) (end 103.124 154.559) (width 0.25) (layer F.Cu) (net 26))
 (segment (start 103.124 154.559) (end 103.124 157.099) (width 0.25) (layer F.Cu) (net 26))
 (segment (start 115.316 154.559) (end 103.124 154.559) (width 0.25) (layer F.Cu) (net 26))
 (segment (start 115.316 162.271) (end 115.316 154.559) (width 0.25) (layer F.Cu) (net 26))
 (segment (start 115.236 163.576) (end 115.236 162.351) (width 0.25) (layer F.Cu) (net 26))
 (segment (start 115.236 162.351) (end 115.316 162.271) (width 0.25) (layer F.Cu) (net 26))
 (segment (start 74.168 138.176) (end 76.2 138.176) (width 0.25) (layer F.Cu) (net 8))
 (segment (start 74.168 159.766) (end 74.168 138.176) (width 0.25) (layer F.Cu) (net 8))
 (segment (start 94.234 156.972) (end 94.234 165.989) (width 0.25) (layer F.Cu) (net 8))
 (segment (start 95.377 156.972) (end 94.234 156.972) (width 0.25) (layer F.Cu) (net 8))
 (segment (start 94.234 165.989) (end 88.9 165.989) (width 0.25) (layer F.Cu) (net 8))
 (segment (start 88.9 165.989) (end 88.9 164.846) (width 0.25) (layer F.Cu) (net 8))
 (segment (start 88.9 164.846) (end 78.74 164.846) (width 0.25) (layer F.Cu) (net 8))
 (segment (start 78.74 159.766) (end 74.168 159.766) (width 0.25) (layer F.Cu) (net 8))
 (segment (start 78.74 164.846) (end 78.74 159.766) (width 0.25) (layer F.Cu) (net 8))
 (segment (start 112.736 163.451) (end 112.736 163.576) (width 0.25) (layer B.Cu) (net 8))
 (segment (start 112.776 161.036) (end 112.736 163.451) (width 0.25) (layer B.Cu) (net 8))
 (segment (start 95.377 156.972) (end 95.377 161.036) (width 0.25) (layer B.Cu) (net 8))
 (segment (start 95.377 161.036) (end 112.776 161.036) (width 0.25) (layer B.Cu) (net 8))
 (segment (start 76.2 145.796) (end 77.851 145.796) (width 0.25) (layer F.Cu) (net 5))
 (segment (start 76.2 158.496) (end 77.851 158.496) (width 0.25) (layer F.Cu) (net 5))
 (segment (start 77.851 152.146) (end 77.851 158.496) (width 0.25) (layer F.Cu) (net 5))
 (segment (start 77.851 145.796) (end 77.851 152.146) (width 0.25) (layer F.Cu) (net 5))
 (segment (start 110.236 162.179) (end 110.236 163.576) (width 0.25) (layer B.Cu) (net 5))
 (segment (start 93.853 162.179) (end 110.236 162.179) (width 0.25) (layer B.Cu) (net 5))
 (segment (start 92.329 159.465) (end 93.853 159.465) (width 0.25) (layer B.Cu) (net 5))
 (segment (start 93.853 159.465) (end 93.853 162.179) (width 0.25) (layer B.Cu) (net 5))
 (segment (start 88.519 152.146) (end 77.888408 152.146) (width 0.25) (layer F.Cu) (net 5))
 (segment (start 88.519 156.845) (end 88.519 152.146) (width 0.25) (layer F.Cu) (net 5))
 (segment (start 92.329 159.465) (end 92.329 156.845) (width 0.25) (layer F.Cu) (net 5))
 (segment (start 92.329 156.845) (end 88.519 156.845) (width 0.25) (layer F.Cu) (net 5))
 (segment (start 110.236 164.651) (end 112.717 167.132) (width 0.25) (layer F.Cu) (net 5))
 (segment (start 110.236 163.576) (end 110.236 164.651) (width 0.25) (layer F.Cu) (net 5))
 (segment (start 112.717 167.132) (end 135.255 167.132) (width 0.25) (layer F.Cu) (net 5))
 (segment (start 135.255 167.132) (end 136.398 165.989) (width 0.25) (layer F.Cu) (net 5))
 (segment (start 136.398 160.782) (end 138.43 158.75) (width 0.25) (layer F.Cu) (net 5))
 (segment (start 136.398 165.989) (end 136.398 160.782) (width 0.25) (layer F.Cu) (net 5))
 (segment (start 98.044 155.312189) (end 98.044 157.099) (width 0.25) (layer F.Cu) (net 17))
 (segment (start 98.035189 155.321) (end 98.044 155.312189) (width 0.25) (layer F.Cu) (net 17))
 (segment (start 89.535 155.321) (end 98.035189 155.321) (width 0.25) (layer F.Cu) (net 17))
 (segment (start 83.82 150.876) (end 89.535 150.876) (width 0.25) (layer F.Cu) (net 17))
 (segment (start 89.535 150.876) (end 89.535 155.321) (width 0.25) (layer F.Cu) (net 17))
 (segment (start 89.281 161.036) (end 83.82 161.036) (width 0.25) (layer B.Cu) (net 30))
 (segment (start 89.281 149.86) (end 89.281 161.036) (width 0.25) (layer B.Cu) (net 30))
 (segment (start 98.298 149.86) (end 89.281 149.86) (width 0.25) (layer B.Cu) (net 30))
 (segment (start 100.584 148.59) (end 98.298 148.59) (width 0.25) (layer B.Cu) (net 30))
 (segment (start 98.298 148.59) (end 98.298 149.86) (width 0.25) (layer B.Cu) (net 30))
 (segment (start 93.98 152.544999) (end 93.98 141.013) (width 0.25) (layer F.Cu) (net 31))
 (segment (start 98.163798 152.534202) (end 93.98 152.544999) (width 0.25) (layer F.Cu) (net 31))
 (segment (start 100.584 151.13) (end 100.584 152.544999) (width 0.25) (layer F.Cu) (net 31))
 (segment (start 100.584 152.544999) (end 98.163798 152.534202) (width 0.25) (layer F.Cu) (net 31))
 (segment (start 93.98 141.013) (end 95.504 140.97) (width 0.25) (layer F.Cu) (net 31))
 (segment (start 88.011 164.846) (end 78.486 164.846) (width 0.25) (layer B.Cu) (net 25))
 (segment (start 78.486 163.581815) (end 76.2 163.576) (width 0.25) (layer B.Cu) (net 25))
 (segment (start 90.932 164.846) (end 88.011 164.846) (width 0.25) (layer B.Cu) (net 25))
 (segment (start 90.932 152.781) (end 90.932 164.719) (width 0.25) (layer B.Cu) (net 31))
 (segment (start 100.584 151.13) (end 100.584 152.781) (width 0.25) (layer B.Cu) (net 31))
 (segment (start 100.584 152.781) (end 90.932 152.781) (width 0.25) (layer B.Cu) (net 31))
 (segment (start 137.550001 161.760001) (end 138.35 162.56) (width 0.25) (layer B.Cu) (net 6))
 (segment (start 136.906 161.116) (end 137.550001 161.760001) (width 0.25) (layer B.Cu) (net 6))
 (segment (start 136.906 156.464) (end 136.906 161.116) (width 0.25) (layer B.Cu) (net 6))
 (segment (start 138.43 154.94) (end 136.906 156.464) (width 0.25) (layer B.Cu) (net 6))
 (segment (start 125.236 163.451) (end 125.236 163.576) (width 0.25) (layer B.Cu) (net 6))
 (segment (start 127.571 161.116) (end 125.236 163.451) (width 0.25) (layer B.Cu) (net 6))
 (segment (start 136.906 161.116) (end 127.571 161.116) (width 0.25) (layer B.Cu) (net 6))
 (segment (start 122.736 163.576) (end 122.936 150.876) (width 0.25) (layer F.Cu) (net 2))
 (segment (start 122.936 150.876) (end 122.936 150.114) (width 0.25) (layer F.Cu) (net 2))
 (segment (start 122.936 150.114) (end 123.19 149.86) (width 0.25) (layer F.Cu) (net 2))
 (segment (start 123.19 149.86) (end 124.587 149.86) (width 0.25) (layer F.Cu) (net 2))
 (segment (start 116.967 149.86) (end 116.967 145.669) (width 0.25) (layer F.Cu) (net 2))
 (segment (start 120.236 156.751) (end 127.127 149.86) (width 0.25) (layer B.Cu) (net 1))
 (segment (start 120.236 163.576) (end 120.236 156.751) (width 0.25) (layer B.Cu) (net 1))
 (segment (start 101.03401 145.8636) (end 100.902205 145.731795) (width 0.25) (layer B.Cu) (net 1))
 (segment (start 101.72841 146.558) (end 101.03401 145.8636) (width 0.25) (layer B.Cu) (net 1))
 (segment (start 127.127 149.86) (end 123.825 146.558) (width 0.25) (layer B.Cu) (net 1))
 (segment (start 123.825 146.558) (end 101.72841 146.558) (width 0.25) (layer B.Cu) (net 1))
 (segment (start 132.66 143.654213) (end 132.66 148.74) (width 0.25) (layer F.Cu) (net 4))
 (segment (start 132.66 142.24) (end 132.66 143.654213) (width 0.25) (layer F.Cu) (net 4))
 (segment (start 130.81 150.59) (end 130.81 154.94) (width 0.25) (layer F.Cu) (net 4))
 (segment (start 132.66 148.74) (end 130.81 150.59) (width 0.25) (layer F.Cu) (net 4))
 (segment (start 130.81 155.929949) (end 130.81 158.75) (width 0.25) (layer F.Cu) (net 4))
 (segment (start 130.81 154.94) (end 130.81 155.929949) (width 0.25) (layer F.Cu) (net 4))
 (segment (start 78.486 163.581815) (end 78.486 164.846) (width 0.25) (layer B.Cu) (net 25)))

